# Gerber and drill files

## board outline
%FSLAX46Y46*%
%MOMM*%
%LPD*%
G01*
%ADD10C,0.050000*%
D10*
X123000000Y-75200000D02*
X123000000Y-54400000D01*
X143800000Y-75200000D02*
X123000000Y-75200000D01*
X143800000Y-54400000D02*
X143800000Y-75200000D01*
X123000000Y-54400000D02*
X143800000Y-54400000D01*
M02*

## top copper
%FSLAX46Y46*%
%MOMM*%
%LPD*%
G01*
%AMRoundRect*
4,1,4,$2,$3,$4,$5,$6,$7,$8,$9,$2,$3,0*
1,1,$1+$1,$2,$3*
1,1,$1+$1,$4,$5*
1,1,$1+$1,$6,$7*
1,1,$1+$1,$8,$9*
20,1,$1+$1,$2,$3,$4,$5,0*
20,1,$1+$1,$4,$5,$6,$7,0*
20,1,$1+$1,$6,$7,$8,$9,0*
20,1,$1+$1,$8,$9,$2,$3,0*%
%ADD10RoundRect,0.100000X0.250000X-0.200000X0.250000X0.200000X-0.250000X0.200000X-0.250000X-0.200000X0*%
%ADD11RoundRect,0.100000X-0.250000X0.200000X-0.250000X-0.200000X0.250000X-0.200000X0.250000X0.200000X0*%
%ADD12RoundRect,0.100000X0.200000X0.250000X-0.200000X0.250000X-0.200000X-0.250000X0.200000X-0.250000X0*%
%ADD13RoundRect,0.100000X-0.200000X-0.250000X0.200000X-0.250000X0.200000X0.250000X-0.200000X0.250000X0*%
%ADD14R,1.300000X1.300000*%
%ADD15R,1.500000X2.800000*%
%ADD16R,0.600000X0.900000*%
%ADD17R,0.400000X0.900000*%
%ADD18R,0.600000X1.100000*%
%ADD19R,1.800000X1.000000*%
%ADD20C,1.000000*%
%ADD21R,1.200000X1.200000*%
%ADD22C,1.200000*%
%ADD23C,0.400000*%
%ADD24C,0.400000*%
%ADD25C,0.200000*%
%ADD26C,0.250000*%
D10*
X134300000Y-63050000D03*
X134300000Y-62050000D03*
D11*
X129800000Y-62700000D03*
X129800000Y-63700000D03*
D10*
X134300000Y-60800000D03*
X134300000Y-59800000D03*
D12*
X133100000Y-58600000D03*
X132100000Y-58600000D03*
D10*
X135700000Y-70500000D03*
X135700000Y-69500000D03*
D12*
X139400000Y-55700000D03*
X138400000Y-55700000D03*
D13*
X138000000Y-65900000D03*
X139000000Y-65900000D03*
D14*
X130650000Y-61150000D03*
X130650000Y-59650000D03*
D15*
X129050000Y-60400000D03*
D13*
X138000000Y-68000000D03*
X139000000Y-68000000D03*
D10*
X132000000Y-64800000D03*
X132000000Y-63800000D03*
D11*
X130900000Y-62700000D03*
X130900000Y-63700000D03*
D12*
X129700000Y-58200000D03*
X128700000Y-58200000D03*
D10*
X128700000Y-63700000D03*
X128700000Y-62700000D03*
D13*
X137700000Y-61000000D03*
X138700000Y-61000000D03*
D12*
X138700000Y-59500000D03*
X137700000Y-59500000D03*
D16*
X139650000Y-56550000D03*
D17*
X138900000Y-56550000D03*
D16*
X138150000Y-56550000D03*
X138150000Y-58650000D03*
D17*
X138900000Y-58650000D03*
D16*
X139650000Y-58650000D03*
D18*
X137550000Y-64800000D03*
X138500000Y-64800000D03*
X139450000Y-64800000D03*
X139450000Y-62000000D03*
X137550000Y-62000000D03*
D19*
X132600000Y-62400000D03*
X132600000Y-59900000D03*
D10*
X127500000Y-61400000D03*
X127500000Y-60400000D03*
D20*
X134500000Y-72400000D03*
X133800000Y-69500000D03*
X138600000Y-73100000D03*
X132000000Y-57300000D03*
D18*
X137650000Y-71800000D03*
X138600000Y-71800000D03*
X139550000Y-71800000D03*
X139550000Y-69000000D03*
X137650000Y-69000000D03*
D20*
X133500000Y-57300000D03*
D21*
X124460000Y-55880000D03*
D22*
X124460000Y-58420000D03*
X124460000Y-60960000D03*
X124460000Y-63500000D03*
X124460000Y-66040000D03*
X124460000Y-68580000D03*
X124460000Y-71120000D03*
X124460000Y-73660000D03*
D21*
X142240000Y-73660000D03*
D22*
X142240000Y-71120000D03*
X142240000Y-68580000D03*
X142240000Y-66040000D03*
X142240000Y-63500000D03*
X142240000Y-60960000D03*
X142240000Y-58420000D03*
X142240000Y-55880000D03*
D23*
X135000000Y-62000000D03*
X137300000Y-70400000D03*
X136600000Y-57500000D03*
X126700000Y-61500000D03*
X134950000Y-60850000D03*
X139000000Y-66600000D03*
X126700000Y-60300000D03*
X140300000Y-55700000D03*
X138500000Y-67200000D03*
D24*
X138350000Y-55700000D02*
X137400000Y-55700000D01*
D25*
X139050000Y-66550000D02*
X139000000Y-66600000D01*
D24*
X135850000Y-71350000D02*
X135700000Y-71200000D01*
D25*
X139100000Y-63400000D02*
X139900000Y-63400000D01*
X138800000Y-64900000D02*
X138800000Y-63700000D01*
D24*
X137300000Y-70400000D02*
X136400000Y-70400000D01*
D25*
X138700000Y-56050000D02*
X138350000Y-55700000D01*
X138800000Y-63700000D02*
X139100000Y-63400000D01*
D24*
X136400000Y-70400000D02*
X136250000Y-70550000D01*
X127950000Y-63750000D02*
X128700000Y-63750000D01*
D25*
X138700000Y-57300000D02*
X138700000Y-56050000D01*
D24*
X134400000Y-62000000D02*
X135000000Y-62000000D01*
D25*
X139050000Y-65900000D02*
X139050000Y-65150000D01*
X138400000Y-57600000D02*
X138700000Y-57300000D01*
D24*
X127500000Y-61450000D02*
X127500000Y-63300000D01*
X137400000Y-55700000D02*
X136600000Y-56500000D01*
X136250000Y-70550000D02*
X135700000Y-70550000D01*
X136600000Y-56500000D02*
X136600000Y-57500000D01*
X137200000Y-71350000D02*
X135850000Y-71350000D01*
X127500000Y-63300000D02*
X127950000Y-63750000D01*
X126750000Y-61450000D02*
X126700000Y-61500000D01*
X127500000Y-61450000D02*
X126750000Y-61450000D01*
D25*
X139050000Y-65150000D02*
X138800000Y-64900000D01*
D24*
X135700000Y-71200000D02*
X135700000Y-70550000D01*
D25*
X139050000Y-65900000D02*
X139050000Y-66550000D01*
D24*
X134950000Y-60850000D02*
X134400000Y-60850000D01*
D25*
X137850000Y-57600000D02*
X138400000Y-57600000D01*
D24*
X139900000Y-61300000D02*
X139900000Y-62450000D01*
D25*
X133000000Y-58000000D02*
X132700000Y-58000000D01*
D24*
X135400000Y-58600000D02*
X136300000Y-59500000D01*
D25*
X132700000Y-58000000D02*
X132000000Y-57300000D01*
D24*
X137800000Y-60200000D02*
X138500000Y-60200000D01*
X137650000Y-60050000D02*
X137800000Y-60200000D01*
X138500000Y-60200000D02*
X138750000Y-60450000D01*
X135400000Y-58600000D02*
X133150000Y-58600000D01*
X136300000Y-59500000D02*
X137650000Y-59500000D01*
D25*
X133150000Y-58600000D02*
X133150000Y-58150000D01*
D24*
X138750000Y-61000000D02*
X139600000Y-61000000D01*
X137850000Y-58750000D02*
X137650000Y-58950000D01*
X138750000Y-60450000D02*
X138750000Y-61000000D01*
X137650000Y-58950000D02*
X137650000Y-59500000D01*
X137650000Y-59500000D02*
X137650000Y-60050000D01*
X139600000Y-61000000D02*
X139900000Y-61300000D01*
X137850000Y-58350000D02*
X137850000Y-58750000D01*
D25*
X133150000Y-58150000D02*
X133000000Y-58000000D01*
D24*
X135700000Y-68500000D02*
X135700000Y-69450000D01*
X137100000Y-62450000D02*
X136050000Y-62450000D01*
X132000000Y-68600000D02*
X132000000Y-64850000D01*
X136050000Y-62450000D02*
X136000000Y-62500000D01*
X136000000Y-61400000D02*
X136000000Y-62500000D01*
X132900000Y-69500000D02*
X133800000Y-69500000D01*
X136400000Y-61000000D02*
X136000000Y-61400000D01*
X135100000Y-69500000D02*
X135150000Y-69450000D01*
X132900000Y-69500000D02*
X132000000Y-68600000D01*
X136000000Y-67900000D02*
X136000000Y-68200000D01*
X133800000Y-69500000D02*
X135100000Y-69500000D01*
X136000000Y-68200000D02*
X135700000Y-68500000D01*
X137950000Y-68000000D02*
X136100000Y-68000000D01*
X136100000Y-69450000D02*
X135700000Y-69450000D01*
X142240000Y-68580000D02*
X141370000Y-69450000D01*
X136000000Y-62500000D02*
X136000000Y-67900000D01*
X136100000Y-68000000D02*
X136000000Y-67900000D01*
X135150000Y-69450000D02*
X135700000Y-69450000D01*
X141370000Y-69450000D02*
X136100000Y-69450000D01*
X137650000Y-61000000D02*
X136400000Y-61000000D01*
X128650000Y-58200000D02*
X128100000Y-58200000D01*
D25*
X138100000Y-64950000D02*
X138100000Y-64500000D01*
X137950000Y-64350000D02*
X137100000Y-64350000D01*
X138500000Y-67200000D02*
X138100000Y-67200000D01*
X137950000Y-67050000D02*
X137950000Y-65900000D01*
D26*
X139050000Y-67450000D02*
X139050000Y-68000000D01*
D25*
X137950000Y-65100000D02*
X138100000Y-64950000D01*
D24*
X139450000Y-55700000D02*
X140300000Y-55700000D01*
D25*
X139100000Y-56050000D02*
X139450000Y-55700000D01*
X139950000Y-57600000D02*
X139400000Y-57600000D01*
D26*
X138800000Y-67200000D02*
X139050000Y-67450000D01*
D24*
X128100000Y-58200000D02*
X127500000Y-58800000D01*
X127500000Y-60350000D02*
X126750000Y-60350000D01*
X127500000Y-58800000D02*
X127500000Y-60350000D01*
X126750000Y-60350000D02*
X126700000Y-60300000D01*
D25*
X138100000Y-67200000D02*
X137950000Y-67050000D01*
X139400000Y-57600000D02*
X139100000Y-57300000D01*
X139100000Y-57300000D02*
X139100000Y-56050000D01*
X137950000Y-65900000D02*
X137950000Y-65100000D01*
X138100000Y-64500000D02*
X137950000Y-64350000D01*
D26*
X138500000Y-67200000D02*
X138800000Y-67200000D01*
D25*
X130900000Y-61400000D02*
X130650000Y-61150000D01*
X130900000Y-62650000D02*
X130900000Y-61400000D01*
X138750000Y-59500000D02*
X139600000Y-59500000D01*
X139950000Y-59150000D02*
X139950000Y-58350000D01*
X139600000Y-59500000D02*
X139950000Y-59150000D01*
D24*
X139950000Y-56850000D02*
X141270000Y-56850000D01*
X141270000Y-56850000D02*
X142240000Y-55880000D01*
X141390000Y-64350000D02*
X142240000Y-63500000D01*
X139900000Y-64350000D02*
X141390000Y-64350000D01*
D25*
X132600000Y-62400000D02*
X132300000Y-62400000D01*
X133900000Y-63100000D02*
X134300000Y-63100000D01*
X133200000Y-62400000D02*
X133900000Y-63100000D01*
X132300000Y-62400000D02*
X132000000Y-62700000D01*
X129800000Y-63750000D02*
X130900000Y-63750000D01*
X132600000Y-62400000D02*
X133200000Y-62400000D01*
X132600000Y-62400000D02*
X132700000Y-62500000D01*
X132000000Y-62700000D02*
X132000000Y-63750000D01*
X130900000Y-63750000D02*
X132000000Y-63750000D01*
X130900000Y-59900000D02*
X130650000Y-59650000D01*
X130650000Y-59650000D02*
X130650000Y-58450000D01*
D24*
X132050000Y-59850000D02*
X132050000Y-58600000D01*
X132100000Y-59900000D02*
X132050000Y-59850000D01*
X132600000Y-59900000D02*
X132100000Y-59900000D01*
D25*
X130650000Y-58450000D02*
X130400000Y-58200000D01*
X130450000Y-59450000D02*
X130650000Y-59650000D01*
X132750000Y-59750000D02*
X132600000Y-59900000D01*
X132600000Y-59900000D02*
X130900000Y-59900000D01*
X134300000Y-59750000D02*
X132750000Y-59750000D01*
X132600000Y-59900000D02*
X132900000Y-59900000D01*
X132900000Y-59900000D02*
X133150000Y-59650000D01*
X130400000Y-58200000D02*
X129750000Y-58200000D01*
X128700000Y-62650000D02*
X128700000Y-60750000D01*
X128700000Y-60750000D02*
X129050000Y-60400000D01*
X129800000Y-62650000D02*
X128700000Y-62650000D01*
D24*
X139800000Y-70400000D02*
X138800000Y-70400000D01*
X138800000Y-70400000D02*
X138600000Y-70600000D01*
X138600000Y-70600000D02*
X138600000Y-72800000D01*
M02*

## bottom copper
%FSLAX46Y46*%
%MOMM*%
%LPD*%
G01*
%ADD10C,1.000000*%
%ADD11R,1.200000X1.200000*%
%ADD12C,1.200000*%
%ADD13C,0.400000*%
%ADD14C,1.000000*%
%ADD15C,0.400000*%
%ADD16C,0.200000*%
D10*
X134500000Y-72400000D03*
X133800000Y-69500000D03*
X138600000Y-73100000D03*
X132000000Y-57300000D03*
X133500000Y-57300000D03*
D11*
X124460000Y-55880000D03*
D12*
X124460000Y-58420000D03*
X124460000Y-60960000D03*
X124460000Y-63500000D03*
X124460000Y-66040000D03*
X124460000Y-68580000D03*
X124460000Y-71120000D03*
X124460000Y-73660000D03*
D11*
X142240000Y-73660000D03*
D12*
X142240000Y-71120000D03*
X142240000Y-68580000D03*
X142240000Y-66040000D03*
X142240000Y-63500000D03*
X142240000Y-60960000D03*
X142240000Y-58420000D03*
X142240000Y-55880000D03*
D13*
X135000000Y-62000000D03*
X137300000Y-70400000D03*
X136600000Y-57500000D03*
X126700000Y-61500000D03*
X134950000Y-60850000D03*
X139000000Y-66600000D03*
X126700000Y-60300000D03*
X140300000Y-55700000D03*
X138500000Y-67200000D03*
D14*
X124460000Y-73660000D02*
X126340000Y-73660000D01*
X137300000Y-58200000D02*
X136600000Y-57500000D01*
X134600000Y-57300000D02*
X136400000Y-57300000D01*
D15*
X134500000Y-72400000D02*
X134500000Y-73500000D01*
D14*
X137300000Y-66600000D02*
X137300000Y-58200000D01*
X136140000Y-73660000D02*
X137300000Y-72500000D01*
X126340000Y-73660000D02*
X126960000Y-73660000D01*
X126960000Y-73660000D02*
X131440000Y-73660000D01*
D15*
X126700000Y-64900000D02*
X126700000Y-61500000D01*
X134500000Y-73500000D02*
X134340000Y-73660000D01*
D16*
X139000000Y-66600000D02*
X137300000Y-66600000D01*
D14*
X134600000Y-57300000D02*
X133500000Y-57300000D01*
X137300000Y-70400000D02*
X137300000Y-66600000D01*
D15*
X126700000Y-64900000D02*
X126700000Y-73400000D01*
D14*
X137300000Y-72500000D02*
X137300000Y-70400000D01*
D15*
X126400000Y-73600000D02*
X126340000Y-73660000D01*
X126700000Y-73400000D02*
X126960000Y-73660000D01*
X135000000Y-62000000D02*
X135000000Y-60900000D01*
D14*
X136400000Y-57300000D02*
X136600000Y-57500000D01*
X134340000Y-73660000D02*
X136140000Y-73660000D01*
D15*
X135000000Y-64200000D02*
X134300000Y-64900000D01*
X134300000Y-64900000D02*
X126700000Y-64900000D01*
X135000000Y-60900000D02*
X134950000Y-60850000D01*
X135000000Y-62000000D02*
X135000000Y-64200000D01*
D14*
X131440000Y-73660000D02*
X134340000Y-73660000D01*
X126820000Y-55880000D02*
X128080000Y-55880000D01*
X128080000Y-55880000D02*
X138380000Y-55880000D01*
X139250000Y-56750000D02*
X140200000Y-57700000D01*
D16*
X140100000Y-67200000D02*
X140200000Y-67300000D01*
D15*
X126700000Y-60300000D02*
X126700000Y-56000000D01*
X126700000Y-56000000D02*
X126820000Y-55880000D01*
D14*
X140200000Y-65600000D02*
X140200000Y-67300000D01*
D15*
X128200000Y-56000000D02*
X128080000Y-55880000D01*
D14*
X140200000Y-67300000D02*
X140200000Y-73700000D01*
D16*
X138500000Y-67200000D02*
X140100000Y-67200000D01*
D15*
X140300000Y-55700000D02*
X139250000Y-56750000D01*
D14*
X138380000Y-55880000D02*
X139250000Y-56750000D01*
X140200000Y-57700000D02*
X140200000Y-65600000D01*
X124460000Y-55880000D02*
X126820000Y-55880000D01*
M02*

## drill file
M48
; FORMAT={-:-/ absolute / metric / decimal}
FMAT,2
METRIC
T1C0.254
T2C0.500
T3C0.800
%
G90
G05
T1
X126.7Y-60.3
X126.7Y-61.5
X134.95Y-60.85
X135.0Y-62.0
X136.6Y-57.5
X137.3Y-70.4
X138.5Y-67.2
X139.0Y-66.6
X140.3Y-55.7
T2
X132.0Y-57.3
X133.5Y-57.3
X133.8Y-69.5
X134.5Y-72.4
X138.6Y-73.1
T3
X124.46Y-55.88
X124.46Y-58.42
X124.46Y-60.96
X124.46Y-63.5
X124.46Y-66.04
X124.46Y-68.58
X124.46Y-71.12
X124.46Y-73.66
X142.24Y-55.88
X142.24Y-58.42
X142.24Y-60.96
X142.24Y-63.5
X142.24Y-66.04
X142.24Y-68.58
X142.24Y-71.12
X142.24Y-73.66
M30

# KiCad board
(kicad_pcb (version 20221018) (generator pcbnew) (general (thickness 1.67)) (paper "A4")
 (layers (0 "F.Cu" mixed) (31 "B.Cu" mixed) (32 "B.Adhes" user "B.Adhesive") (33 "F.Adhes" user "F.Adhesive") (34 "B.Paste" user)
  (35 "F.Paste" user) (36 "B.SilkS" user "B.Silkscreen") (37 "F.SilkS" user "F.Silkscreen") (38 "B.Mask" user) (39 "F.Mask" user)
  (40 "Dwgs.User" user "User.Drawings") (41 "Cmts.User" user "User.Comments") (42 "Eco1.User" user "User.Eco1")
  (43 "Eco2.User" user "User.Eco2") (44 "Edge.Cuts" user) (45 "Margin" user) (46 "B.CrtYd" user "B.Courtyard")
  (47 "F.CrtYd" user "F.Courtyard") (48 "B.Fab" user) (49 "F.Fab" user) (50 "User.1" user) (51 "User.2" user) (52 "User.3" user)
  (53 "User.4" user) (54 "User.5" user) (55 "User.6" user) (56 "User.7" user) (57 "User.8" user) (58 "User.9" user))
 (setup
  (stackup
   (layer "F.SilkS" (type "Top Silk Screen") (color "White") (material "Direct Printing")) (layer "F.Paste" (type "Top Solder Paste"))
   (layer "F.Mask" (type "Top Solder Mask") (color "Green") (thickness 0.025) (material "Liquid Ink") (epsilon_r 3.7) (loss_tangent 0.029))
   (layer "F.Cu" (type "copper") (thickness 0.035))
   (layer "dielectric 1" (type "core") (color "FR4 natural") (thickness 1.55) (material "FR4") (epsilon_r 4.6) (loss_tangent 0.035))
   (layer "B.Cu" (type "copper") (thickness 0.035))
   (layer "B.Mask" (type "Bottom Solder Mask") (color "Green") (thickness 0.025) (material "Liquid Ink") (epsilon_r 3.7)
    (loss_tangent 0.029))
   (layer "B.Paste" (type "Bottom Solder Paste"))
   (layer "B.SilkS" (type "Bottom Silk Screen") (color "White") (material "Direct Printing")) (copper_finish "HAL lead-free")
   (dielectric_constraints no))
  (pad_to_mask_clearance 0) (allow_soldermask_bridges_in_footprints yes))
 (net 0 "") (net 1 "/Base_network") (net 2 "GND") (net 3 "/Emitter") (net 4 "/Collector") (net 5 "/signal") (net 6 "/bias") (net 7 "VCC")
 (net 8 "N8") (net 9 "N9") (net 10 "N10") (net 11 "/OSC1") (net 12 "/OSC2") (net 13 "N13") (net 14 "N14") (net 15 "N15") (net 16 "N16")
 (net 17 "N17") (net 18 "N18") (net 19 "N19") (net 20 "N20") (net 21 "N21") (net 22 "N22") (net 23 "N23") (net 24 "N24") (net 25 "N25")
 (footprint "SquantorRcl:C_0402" (layer "F.Cu") (at 134.3 62.55 90)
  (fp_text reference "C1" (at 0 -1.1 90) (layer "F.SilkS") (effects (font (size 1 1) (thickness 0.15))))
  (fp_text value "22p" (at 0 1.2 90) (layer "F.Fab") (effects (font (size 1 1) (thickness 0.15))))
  (pad "1" smd roundrect (at -0.5 0 90) (size 0.6 0.7) (layers "F.Cu" "F.Paste" "F.Mask") (roundrect_rratio 0.1666666667)
   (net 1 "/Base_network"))
  (pad "2" smd roundrect (at 0.5 0 90) (size 0.6 0.7) (layers "F.Cu" "F.Paste" "F.Mask") (roundrect_rratio 0.1666666667) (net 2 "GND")))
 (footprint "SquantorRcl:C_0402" (layer "F.Cu") (at 129.8 63.2 -90)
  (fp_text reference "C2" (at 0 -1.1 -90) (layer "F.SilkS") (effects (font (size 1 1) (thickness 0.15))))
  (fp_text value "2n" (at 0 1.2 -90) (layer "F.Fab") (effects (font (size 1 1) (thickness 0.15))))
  (pad "1" smd roundrect (at -0.5 0 270) (size 0.6 0.7) (layers "F.Cu" "F.Paste" "F.Mask") (roundrect_rratio 0.1666666667)
   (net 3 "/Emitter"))
  (pad "2" smd roundrect (at 0.5 0 270) (size 0.6 0.7) (layers "F.Cu" "F.Paste" "F.Mask") (roundrect_rratio 0.1666666667)
   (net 1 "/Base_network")))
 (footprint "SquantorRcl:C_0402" (layer "F.Cu") (at 134.3 60.3 90)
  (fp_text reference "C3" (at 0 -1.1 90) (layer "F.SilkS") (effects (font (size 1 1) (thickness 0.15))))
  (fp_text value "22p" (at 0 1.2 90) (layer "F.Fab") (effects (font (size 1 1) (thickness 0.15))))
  (pad "1" smd roundrect (at -0.5 0 90) (size 0.6 0.7) (layers "F.Cu" "F.Paste" "F.Mask") (roundrect_rratio 0.1666666667) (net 2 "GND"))
  (pad "2" smd roundrect (at 0.5 0 90) (size 0.6 0.7) (layers "F.Cu" "F.Paste" "F.Mask") (roundrect_rratio 0.1666666667)
   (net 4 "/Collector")))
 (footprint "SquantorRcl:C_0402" (layer "F.Cu") (at 132.6 58.6 180)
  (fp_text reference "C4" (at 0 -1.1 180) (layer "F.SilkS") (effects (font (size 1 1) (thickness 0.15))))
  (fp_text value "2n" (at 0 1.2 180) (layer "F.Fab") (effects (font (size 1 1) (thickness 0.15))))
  (pad "1" smd roundrect (at -0.5 0 180) (size 0.6 0.7) (layers "F.Cu" "F.Paste" "F.Mask") (roundrect_rratio 0.1666666667) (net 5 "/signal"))
  (pad "2" smd roundrect (at 0.5 0 180) (size 0.6 0.7) (layers "F.Cu" "F.Paste" "F.Mask") (roundrect_rratio 0.1666666667)
   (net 4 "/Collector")))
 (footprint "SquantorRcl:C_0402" (layer "F.Cu") (at 135.7 70 90)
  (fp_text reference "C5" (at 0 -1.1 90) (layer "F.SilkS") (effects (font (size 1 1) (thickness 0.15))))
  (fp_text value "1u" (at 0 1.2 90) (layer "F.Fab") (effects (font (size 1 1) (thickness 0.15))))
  (pad "1" smd roundrect (at -0.5 0 90) (size 0.6 0.7) (layers "F.Cu" "F.Paste" "F.Mask") (roundrect_rratio 0.1666666667) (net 2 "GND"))
  (pad "2" smd roundrect (at 0.5 0 90) (size 0.6 0.7) (layers "F.Cu" "F.Paste" "F.Mask") (roundrect_rratio 0.1666666667) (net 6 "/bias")))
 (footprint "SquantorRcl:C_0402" (layer "F.Cu") (at 138.9 55.7 180)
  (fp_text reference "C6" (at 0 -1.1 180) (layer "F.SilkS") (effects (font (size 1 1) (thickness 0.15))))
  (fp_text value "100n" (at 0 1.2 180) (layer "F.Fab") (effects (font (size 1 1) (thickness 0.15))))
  (pad "1" smd roundrect (at -0.5 0 180) (size 0.6 0.7) (layers "F.Cu" "F.Paste" "F.Mask") (roundrect_rratio 0.1666666667) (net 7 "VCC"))
  (pad "2" smd roundrect (at 0.5 0 180) (size 0.6 0.7) (layers "F.Cu" "F.Paste" "F.Mask") (roundrect_rratio 0.1666666667) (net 2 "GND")))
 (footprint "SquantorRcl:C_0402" (layer "F.Cu") (at 138.5 65.9)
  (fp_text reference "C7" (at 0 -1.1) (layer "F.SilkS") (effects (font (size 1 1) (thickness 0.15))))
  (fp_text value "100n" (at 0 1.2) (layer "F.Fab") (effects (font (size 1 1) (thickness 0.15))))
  (pad "1" smd roundrect (at -0.5 0) (size 0.6 0.7) (layers "F.Cu" "F.Paste" "F.Mask") (roundrect_rratio 0.1666666667) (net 7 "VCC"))
  (pad "2" smd roundrect (at 0.5 0) (size 0.6 0.7) (layers "F.Cu" "F.Paste" "F.Mask") (roundrect_rratio 0.1666666667) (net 2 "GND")))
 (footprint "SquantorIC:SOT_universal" (layer "F.Cu") (at 129.9 60.4 90)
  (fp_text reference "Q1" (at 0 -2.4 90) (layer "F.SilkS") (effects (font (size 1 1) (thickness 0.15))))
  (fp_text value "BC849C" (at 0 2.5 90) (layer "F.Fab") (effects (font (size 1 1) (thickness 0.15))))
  (pad "1" smd rect (at -0.75 0.75 90) (size 1.3 1.3) (layers "F.Cu" "F.Paste" "F.Mask") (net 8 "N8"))
  (pad "2" smd rect (at 0.75 0.75 90) (size 1.3 1.3) (layers "F.Cu" "F.Paste" "F.Mask") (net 4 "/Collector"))
  (pad "3" smd rect (at 0 -0.85 90) (size 2.8 1.5) (layers "F.Cu" "F.Paste" "F.Mask") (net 3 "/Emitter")))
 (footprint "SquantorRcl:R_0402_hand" (layer "F.Cu") (at 138.5 68)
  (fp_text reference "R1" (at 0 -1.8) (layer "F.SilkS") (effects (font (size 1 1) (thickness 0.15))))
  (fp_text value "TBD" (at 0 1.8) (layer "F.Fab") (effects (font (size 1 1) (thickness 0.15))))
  (pad "1" smd roundrect (at -0.5 0) (size 0.6 0.7) (layers "F.Cu" "F.Paste" "F.Mask") (roundrect_rratio 0.1666666667) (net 6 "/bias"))
  (pad "2" smd roundrect (at 0.5 0) (size 0.6 0.7) (layers "F.Cu" "F.Paste" "F.Mask") (roundrect_rratio 0.1666666667) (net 7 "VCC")))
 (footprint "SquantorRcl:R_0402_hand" (layer "F.Cu") (at 132 64.3 90)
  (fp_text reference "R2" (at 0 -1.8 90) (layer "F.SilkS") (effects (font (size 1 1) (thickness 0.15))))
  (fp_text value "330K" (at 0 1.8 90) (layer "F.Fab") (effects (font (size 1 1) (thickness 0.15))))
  (pad "1" smd roundrect (at -0.5 0 90) (size 0.6 0.7) (layers "F.Cu" "F.Paste" "F.Mask") (roundrect_rratio 0.1666666667) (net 6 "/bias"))
  (pad "2" smd roundrect (at 0.5 0 90) (size 0.6 0.7) (layers "F.Cu" "F.Paste" "F.Mask") (roundrect_rratio 0.1666666667)
   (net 1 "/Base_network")))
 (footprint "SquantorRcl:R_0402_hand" (layer "F.Cu") (at 130.9 63.2 -90)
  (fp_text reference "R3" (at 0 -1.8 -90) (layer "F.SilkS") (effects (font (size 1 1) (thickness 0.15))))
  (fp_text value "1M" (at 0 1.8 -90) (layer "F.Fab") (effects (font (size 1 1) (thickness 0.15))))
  (pad "1" smd roundrect (at -0.5 0 270) (size 0.6 0.7) (layers "F.Cu" "F.Paste" "F.Mask") (roundrect_rratio 0.1666666667) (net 8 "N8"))
  (pad "2" smd roundrect (at 0.5 0 270) (size 0.6 0.7) (layers "F.Cu" "F.Paste" "F.Mask") (roundrect_rratio 0.1666666667)
   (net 1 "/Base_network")))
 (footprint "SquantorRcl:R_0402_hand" (layer "F.Cu") (at 129.2 58.2 180)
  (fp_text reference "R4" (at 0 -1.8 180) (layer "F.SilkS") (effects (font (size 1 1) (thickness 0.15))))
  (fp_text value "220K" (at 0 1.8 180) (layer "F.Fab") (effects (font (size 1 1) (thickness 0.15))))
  (pad "1" smd roundrect (at -0.5 0 180) (size 0.6 0.7) (layers "F.Cu" "F.Paste" "F.Mask") (roundrect_rratio 0.1666666667)
   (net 4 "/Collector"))
  (pad "2" smd roundrect (at 0.5 0 180) (size 0.6 0.7) (layers "F.Cu" "F.Paste" "F.Mask") (roundrect_rratio 0.1666666667) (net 7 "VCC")))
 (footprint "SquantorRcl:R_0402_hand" (layer "F.Cu") (at 128.7 63.2 90)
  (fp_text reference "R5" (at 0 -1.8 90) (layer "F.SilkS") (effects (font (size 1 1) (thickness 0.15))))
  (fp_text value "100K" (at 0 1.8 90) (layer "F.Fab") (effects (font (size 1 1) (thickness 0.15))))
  (pad "1" smd roundrect (at -0.5 0 90) (size 0.6 0.7) (layers "F.Cu" "F.Paste" "F.Mask") (roundrect_rratio 0.1666666667) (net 2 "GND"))
  (pad "2" smd roundrect (at 0.5 0 90) (size 0.6 0.7) (layers "F.Cu" "F.Paste" "F.Mask") (roundrect_rratio 0.1666666667) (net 3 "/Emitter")))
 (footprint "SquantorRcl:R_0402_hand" (layer "F.Cu") (at 138.2 61)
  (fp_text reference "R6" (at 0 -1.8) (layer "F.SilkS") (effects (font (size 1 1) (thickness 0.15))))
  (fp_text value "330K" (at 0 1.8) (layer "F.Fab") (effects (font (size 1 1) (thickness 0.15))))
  (pad "1" smd roundrect (at -0.5 0) (size 0.6 0.7) (layers "F.Cu" "F.Paste" "F.Mask") (roundrect_rratio 0.1666666667) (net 6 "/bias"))
  (pad "2" smd roundrect (at 0.5 0) (size 0.6 0.7) (layers "F.Cu" "F.Paste" "F.Mask") (roundrect_rratio 0.1666666667) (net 5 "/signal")))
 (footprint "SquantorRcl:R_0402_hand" (layer "F.Cu") (at 138.2 59.5 180)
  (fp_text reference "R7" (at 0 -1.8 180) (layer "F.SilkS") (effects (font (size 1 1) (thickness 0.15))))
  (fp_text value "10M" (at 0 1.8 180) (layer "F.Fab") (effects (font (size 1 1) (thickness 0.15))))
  (pad "1" smd roundrect (at -0.5 0 180) (size 0.6 0.7) (layers "F.Cu" "F.Paste" "F.Mask") (roundrect_rratio 0.1666666667) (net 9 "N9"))
  (pad "2" smd roundrect (at 0.5 0 180) (size 0.6 0.7) (layers "F.Cu" "F.Paste" "F.Mask") (roundrect_rratio 0.1666666667) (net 5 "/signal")))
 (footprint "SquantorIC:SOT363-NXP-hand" (layer "F.Cu") (at 138.9 57.6 -90)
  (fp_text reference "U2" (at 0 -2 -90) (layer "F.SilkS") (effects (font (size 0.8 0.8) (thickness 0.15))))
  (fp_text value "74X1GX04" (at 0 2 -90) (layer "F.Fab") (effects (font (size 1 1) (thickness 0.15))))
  (pad "1" smd rect (at -1.05 -0.75 180) (size 0.6 0.9) (layers "F.Cu" "F.Paste" "F.Mask") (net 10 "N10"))
  (pad "2" smd rect (at -1.05 0 180) (size 0.4 0.9) (layers "F.Cu" "F.Paste" "F.Mask") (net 2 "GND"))
  (pad "3" smd rect (at -1.05 0.75 180) (size 0.6 0.9) (layers "F.Cu" "F.Paste" "F.Mask") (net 5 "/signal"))
  (pad "4" smd rect (at 1.05 0.75 180) (size 0.6 0.9) (layers "F.Cu" "F.Paste" "F.Mask") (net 9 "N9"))
  (pad "5" smd rect (at 1.05 0 180) (size 0.4 0.9) (layers "F.Cu" "F.Paste" "F.Mask") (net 7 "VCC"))
  (pad "6" smd rect (at 1.05 -0.75 180) (size 0.6 0.9) (layers "F.Cu" "F.Paste" "F.Mask") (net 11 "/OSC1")))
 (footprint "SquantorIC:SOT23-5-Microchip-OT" (layer "F.Cu") (at 138.5 63.4 90)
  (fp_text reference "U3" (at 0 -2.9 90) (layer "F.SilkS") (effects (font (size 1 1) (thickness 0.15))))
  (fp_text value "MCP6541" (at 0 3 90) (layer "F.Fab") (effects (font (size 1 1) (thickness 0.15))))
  (pad "1" smd rect (at -1.4 -0.95) (size 0.6 1.1) (layers "F.Cu" "F.Paste" "F.Mask") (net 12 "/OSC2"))
  (pad "2" smd rect (at -1.4 0) (size 0.6 1.1) (layers "F.Cu" "F.Paste" "F.Mask") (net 2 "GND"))
  (pad "3" smd rect (at -1.4 0.95) (size 0.6 1.1) (layers "F.Cu" "F.Paste" "F.Mask") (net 5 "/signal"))
  (pad "4" smd rect (at 1.4 0.95) (size 0.6 1.1) (layers "F.Cu" "F.Paste" "F.Mask") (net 6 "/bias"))
  (pad "5" smd rect (at 1.4 -0.95) (size 0.6 1.1) (layers "F.Cu" "F.Paste" "F.Mask") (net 7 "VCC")))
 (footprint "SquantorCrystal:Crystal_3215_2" (layer "F.Cu") (at 132.6 61.15 90)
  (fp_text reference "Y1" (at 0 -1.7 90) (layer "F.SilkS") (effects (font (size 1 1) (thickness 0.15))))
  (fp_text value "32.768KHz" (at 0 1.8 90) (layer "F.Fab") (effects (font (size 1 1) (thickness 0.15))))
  (pad "1" smd rect (at -1.25 0 90) (size 1 1.8) (layers "F.Cu" "F.Paste" "F.Mask") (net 1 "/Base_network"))
  (pad "2" smd rect (at 1.25 0 90) (size 1 1.8) (layers "F.Cu" "F.Paste" "F.Mask") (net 4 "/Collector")))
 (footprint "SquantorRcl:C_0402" (layer "F.Cu") (at 127.5 60.9 90)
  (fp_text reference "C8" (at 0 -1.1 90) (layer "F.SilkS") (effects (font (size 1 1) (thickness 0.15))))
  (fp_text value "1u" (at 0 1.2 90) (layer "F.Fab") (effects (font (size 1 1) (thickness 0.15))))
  (pad "1" smd roundrect (at -0.5 0 90) (size 0.6 0.7) (layers "F.Cu" "F.Paste" "F.Mask") (roundrect_rratio 0.1666666667) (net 2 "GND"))
  (pad "2" smd roundrect (at 0.5 0 90) (size 0.6 0.7) (layers "F.Cu" "F.Paste" "F.Mask") (roundrect_rratio 0.1666666667) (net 7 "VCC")))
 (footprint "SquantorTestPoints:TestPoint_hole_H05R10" (layer "F.Cu") (at 134.5 72.4)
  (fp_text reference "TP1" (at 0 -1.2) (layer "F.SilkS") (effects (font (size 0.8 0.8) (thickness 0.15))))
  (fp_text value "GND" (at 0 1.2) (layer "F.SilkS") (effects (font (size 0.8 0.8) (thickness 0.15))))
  (pad "1" thru_hole circle (at 0 0) (size 1 1) (drill 0.5) (layers "*.Cu" "*.Mask") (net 2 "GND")))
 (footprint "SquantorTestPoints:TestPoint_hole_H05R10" (layer "F.Cu") (at 133.8 69.5)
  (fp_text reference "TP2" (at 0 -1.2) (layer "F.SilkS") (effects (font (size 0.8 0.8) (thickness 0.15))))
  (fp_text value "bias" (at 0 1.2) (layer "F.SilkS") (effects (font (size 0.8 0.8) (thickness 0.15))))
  (pad "1" thru_hole circle (at 0 0) (size 1 1) (drill 0.5) (layers "*.Cu" "*.Mask") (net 6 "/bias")))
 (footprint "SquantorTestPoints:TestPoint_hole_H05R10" (layer "F.Cu") (at 138.6 73.1)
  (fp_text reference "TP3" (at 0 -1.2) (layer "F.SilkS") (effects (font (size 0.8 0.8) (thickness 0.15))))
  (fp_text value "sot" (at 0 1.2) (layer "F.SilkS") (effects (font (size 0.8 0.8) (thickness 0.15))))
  (pad "1" thru_hole circle (at 0 0) (size 1 1) (drill 0.5) (layers "*.Cu" "*.Mask") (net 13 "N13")))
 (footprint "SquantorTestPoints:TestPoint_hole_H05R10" (layer "F.Cu") (at 132 57.3)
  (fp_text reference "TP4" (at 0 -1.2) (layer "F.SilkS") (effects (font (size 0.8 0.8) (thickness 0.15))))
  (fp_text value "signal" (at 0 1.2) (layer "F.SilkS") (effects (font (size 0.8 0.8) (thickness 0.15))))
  (pad "1" thru_hole circle (at 0 0) (size 1 1) (drill 0.5) (layers "*.Cu" "*.Mask") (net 5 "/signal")))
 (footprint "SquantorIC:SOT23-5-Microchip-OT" (layer "F.Cu") (at 138.6 70.4 90)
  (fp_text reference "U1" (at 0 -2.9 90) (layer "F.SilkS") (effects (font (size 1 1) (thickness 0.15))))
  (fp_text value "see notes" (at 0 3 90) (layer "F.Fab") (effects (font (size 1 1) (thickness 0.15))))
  (pad "1" smd rect (at -1.4 -0.95) (size 0.6 1.1) (layers "F.Cu" "F.Paste" "F.Mask") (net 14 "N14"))
  (pad "2" smd rect (at -1.4 0) (size 0.6 1.1) (layers "F.Cu" "F.Paste" "F.Mask") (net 13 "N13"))
  (pad "3" smd rect (at -1.4 0.95) (size 0.6 1.1) (layers "F.Cu" "F.Paste" "F.Mask") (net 6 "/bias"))
  (pad "4" smd rect (at 1.4 0.95) (size 0.6 1.1) (layers "F.Cu" "F.Paste" "F.Mask") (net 6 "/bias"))
  (pad "5" smd rect (at 1.4 -0.95) (size 0.6 1.1) (layers "F.Cu" "F.Paste" "F.Mask") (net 2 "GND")))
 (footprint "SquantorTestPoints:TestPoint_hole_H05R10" (layer "F.Cu") (at 133.5 57.3)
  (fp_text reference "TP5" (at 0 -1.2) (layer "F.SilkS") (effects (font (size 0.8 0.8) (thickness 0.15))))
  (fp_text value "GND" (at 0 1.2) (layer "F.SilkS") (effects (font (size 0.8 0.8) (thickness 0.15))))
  (pad "1" thru_hole circle (at 0 0) (size 1 1) (drill 0.5) (layers "*.Cu" "*.Mask") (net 2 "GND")))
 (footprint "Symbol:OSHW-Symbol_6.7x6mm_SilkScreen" (layer "B.Cu") (at 134.27 64.77 180)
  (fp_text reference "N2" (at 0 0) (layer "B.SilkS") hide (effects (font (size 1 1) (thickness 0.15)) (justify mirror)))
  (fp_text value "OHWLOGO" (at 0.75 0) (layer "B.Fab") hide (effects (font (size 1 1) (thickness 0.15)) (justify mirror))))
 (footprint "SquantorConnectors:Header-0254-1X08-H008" (layer "B.Cu") (at 124.46 64.77 -90)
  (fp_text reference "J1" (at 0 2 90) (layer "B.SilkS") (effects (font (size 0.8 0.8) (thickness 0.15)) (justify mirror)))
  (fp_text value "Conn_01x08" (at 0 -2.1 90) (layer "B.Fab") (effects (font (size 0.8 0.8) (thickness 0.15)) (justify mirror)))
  (pad "1" thru_hole rect (at -8.89 0 90) (size 1.2 1.2) (drill 0.8) (layers "*.Cu" "*.Mask") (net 7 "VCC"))
  (pad "2" thru_hole circle (at -6.35 0 90) (size 1.2 1.2) (drill 0.8) (layers "*.Cu" "*.Mask") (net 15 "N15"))
  (pad "3" thru_hole circle (at -3.81 0 90) (size 1.2 1.2) (drill 0.8) (layers "*.Cu" "*.Mask") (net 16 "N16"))
  (pad "4" thru_hole circle (at -1.27 0 90) (size 1.2 1.2) (drill 0.8) (layers "*.Cu" "*.Mask") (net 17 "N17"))
  (pad "5" thru_hole circle (at 1.27 0 90) (size 1.2 1.2) (drill 0.8) (layers "*.Cu" "*.Mask") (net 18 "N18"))
  (pad "6" thru_hole circle (at 3.81 0 90) (size 1.2 1.2) (drill 0.8) (layers "*.Cu" "*.Mask") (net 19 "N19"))
  (pad "7" thru_hole circle (at 6.35 0 90) (size 1.2 1.2) (drill 0.8) (layers "*.Cu" "*.Mask") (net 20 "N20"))
  (pad "8" thru_hole circle (at 8.89 0 90) (size 1.2 1.2) (drill 0.8) (layers "*.Cu" "*.Mask") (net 2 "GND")))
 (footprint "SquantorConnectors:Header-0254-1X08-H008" (layer "B.Cu") (at 142.24 64.77 90)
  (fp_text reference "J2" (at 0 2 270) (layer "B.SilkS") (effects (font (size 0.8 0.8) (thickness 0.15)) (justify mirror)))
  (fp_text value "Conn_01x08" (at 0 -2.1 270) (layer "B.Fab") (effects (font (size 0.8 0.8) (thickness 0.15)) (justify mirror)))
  (pad "1" thru_hole rect (at -8.89 0 270) (size 1.2 1.2) (drill 0.8) (layers "*.Cu" "*.Mask") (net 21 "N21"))
  (pad "2" thru_hole circle (at -6.35 0 270) (size 1.2 1.2) (drill 0.8) (layers "*.Cu" "*.Mask") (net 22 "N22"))
  (pad "3" thru_hole circle (at -3.81 0 270) (size 1.2 1.2) (drill 0.8) (layers "*.Cu" "*.Mask") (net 6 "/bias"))
  (pad "4" thru_hole circle (at -1.27 0 270) (size 1.2 1.2) (drill 0.8) (layers "*.Cu" "*.Mask") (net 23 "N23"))
  (pad "5" thru_hole circle (at 1.27 0 270) (size 1.2 1.2) (drill 0.8) (layers "*.Cu" "*.Mask") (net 12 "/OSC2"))
  (pad "6" thru_hole circle (at 3.81 0 270) (size 1.2 1.2) (drill 0.8) (layers "*.Cu" "*.Mask") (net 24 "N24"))
  (pad "7" thru_hole circle (at 6.35 0 270) (size 1.2 1.2) (drill 0.8) (layers "*.Cu" "*.Mask") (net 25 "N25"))
  (pad "8" thru_hole circle (at 8.89 0 270) (size 1.2 1.2) (drill 0.8) (layers "*.Cu" "*.Mask") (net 11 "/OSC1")))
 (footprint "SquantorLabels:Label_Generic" (layer "B.Cu") (at 134.97 68.3 180)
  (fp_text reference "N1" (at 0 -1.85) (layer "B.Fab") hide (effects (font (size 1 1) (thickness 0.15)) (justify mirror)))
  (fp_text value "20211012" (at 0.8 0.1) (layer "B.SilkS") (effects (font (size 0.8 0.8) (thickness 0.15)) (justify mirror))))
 (gr_line (start 123 75.2) (end 123 54.4) (stroke (width 0.05) (type solid)) (layer "Edge.Cuts"))
 (gr_line (start 143.8 75.2) (end 123 75.2) (stroke (width 0.05) (type solid)) (layer "Edge.Cuts"))
 (gr_line (start 143.8 54.4) (end 143.8 75.2) (stroke (width 0.05) (type solid)) (layer "Edge.Cuts"))
 (gr_line (start 123 54.4) (end 143.8 54.4) (stroke (width 0.05) (type solid)) (layer "Edge.Cuts"))
 (segment (start 138.35 55.7) (end 137.4 55.7) (width 0.4) (layer "F.Cu") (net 2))
 (segment (start 139.05 66.55) (end 139 66.6) (width 0.2) (layer "F.Cu") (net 2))
 (segment (start 135.85 71.35) (end 135.7 71.2) (width 0.4) (layer "F.Cu") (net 2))
 (segment (start 139.1 63.4) (end 139.9 63.4) (width 0.2) (layer "F.Cu") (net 2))
 (segment (start 138.8 64.9) (end 138.8 63.7) (width 0.2) (layer "F.Cu") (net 2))
 (segment (start 137.3 70.4) (end 136.4 70.4) (width 0.4) (layer "F.Cu") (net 2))
 (segment (start 138.7 56.05) (end 138.35 55.7) (width 0.2) (layer "F.Cu") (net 2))
 (segment (start 138.8 63.7) (end 139.1 63.4) (width 0.2) (layer "F.Cu") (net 2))
 (segment (start 136.4 70.4) (end 136.25 70.55) (width 0.4) (layer "F.Cu") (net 2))
 (segment (start 127.95 63.75) (end 128.7 63.75) (width 0.4) (layer "F.Cu") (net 2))
 (segment (start 138.7 57.3) (end 138.7 56.05) (width 0.2) (layer "F.Cu") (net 2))
 (segment (start 134.4 62) (end 135 62) (width 0.4) (layer "F.Cu") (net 2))
 (segment (start 139.05 65.9) (end 139.05 65.15) (width 0.2) (layer "F.Cu") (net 2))
 (segment (start 138.4 57.6) (end 138.7 57.3) (width 0.2) (layer "F.Cu") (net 2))
 (segment (start 127.5 61.45) (end 127.5 63.3) (width 0.4) (layer "F.Cu") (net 2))
 (segment (start 137.4 55.7) (end 136.6 56.5) (width 0.4) (layer "F.Cu") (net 2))
 (segment (start 136.25 70.55) (end 135.7 70.55) (width 0.4) (layer "F.Cu") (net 2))
 (segment (start 136.6 56.5) (end 136.6 57.5) (width 0.4) (layer "F.Cu") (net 2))
 (segment (start 137.2 71.35) (end 135.85 71.35) (width 0.4) (layer "F.Cu") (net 2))
 (segment (start 127.5 63.3) (end 127.95 63.75) (width 0.4) (layer "F.Cu") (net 2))
 (segment (start 126.75 61.45) (end 126.7 61.5) (width 0.4) (layer "F.Cu") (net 2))
 (segment (start 127.5 61.45) (end 126.75 61.45) (width 0.4) (layer "F.Cu") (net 2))
 (segment (start 139.05 65.15) (end 138.8 64.9) (width 0.2) (layer "F.Cu") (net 2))
 (segment (start 135.7 71.2) (end 135.7 70.55) (width 0.4) (layer "F.Cu") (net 2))
 (segment (start 139.05 65.9) (end 139.05 66.55) (width 0.2) (layer "F.Cu") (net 2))
 (segment (start 134.95 60.85) (end 134.4 60.85) (width 0.4) (layer "F.Cu") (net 2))
 (segment (start 137.85 57.6) (end 138.4 57.6) (width 0.2) (layer "F.Cu") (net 2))
 (via (at 135 62) (size 0.4) (drill 0.254) (layers "F.Cu" "B.Cu") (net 2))
 (via (at 137.3 70.4) (size 0.4) (drill 0.254) (layers "F.Cu" "B.Cu") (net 2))
 (via (at 136.6 57.5) (size 0.4) (drill 0.254) (layers "F.Cu" "B.Cu") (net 2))
 (via (at 126.7 61.5) (size 0.4) (drill 0.254) (layers "F.Cu" "B.Cu") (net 2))
 (via (at 134.95 60.85) (size 0.4) (drill 0.254) (layers "F.Cu" "B.Cu") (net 2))
 (via (at 139 66.6) (size 0.4) (drill 0.254) (layers "F.Cu" "B.Cu") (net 2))
 (segment (start 124.46 73.66) (end 126.34 73.66) (width 1) (layer "B.Cu") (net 2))
 (segment (start 137.3 58.2) (end 136.6 57.5) (width 1) (layer "B.Cu") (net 2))
 (segment (start 134.6 57.3) (end 136.4 57.3) (width 1) (layer "B.Cu") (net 2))
 (segment (start 134.5 72.4) (end 134.5 73.5) (width 0.4) (layer "B.Cu") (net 2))
 (segment (start 137.3 66.6) (end 137.3 58.2) (width 1) (layer "B.Cu") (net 2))
 (segment (start 136.14 73.66) (end 137.3 72.5) (width 1) (layer "B.Cu") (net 2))
 (segment (start 126.34 73.66) (end 126.96 73.66) (width 1) (layer "B.Cu") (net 2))
 (segment (start 126.96 73.66) (end 131.44 73.66) (width 1) (layer "B.Cu") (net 2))
 (segment (start 126.7 64.9) (end 126.7 61.5) (width 0.4) (layer "B.Cu") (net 2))
 (segment (start 134.5 73.5) (end 134.34 73.66) (width 0.4) (layer "B.Cu") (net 2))
 (segment (start 139 66.6) (end 137.3 66.6) (width 0.2) (layer "B.Cu") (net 2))
 (segment (start 134.6 57.3) (end 133.5 57.3) (width 1) (layer "B.Cu") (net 2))
 (segment (start 137.3 70.4) (end 137.3 66.6) (width 1) (layer "B.Cu") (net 2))
 (segment (start 126.7 64.9) (end 126.7 73.4) (width 0.4) (layer "B.Cu") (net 2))
 (segment (start 137.3 72.5) (end 137.3 70.4) (width 1) (layer "B.Cu") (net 2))
 (segment (start 126.4 73.6) (end 126.34 73.66) (width 0.4) (layer "B.Cu") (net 2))
 (segment (start 126.7 73.4) (end 126.96 73.66) (width 0.4) (layer "B.Cu") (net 2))
 (segment (start 135 62) (end 135 60.9) (width 0.4) (layer "B.Cu") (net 2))
 (segment (start 136.4 57.3) (end 136.6 57.5) (width 1) (layer "B.Cu") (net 2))
 (segment (start 134.34 73.66) (end 136.14 73.66) (width 1) (layer "B.Cu") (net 2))
 (segment (start 135 64.2) (end 134.3 64.9) (width 0.4) (layer "B.Cu") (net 2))
 (segment (start 134.3 64.9) (end 126.7 64.9) (width 0.4) (layer "B.Cu") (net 2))
 (segment (start 135 60.9) (end 134.95 60.85) (width 0.4) (layer "B.Cu") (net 2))
 (segment (start 135 62) (end 135 64.2) (width 0.4) (layer "B.Cu") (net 2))
 (segment (start 131.44 73.66) (end 134.34 73.66) (width 1) (layer "B.Cu") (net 2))
 (segment (start 139.9 61.3) (end 139.9 62.45) (width 0.4) (layer "F.Cu") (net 5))
 (segment (start 133 58) (end 132.7 58) (width 0.2) (layer "F.Cu") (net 5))
 (segment (start 135.4 58.6) (end 136.3 59.5) (width 0.4) (layer "F.Cu") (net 5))
 (segment (start 132.7 58) (end 132 57.3) (width 0.2) (layer "F.Cu") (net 5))
 (segment (start 137.8 60.2) (end 138.5 60.2) (width 0.4) (layer "F.Cu") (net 5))
 (segment (start 137.65 60.05) (end 137.8 60.2) (width 0.4) (layer "F.Cu") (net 5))
 (segment (start 138.5 60.2) (end 138.75 60.45) (width 0.4) (layer "F.Cu") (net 5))
 (segment (start 135.4 58.6) (end 133.15 58.6) (width 0.4) (layer "F.Cu") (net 5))
 (segment (start 136.3 59.5) (end 137.65 59.5) (width 0.4) (layer "F.Cu") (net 5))
 (segment (start 133.15 58.6) (end 133.15 58.15) (width 0.2) (layer "F.Cu") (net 5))
 (segment (start 138.75 61) (end 139.6 61) (width 0.4) (layer "F.Cu") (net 5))
 (segment (start 137.85 58.75) (end 137.65 58.95) (width 0.4) (layer "F.Cu") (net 5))
 (segment (start 138.75 60.45) (end 138.75 61) (width 0.4) (layer "F.Cu") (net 5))
 (segment (start 137.65 58.95) (end 137.65 59.5) (width 0.4) (layer "F.Cu") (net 5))
 (segment (start 137.65 59.5) (end 137.65 60.05) (width 0.4) (layer "F.Cu") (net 5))
 (segment (start 139.6 61) (end 139.9 61.3) (width 0.4) (layer "F.Cu") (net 5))
 (segment (start 137.85 58.35) (end 137.85 58.75) (width 0.4) (layer "F.Cu") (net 5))
 (segment (start 133.15 58.15) (end 133 58) (width 0.2) (layer "F.Cu") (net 5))
 (segment (start 135.7 68.5) (end 135.7 69.45) (width 0.4) (layer "F.Cu") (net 6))
 (segment (start 137.1 62.45) (end 136.05 62.45) (width 0.4) (layer "F.Cu") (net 6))
 (segment (start 132 68.6) (end 132 64.85) (width 0.4) (layer "F.Cu") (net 6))
 (segment (start 136.05 62.45) (end 136 62.5) (width 0.4) (layer "F.Cu") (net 6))
 (segment (start 136 61.4) (end 136 62.5) (width 0.4) (layer "F.Cu") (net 6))
 (segment (start 132.9 69.5) (end 133.8 69.5) (width 0.4) (layer "F.Cu") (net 6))
 (segment (start 136.4 61) (end 136 61.4) (width 0.4) (layer "F.Cu") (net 6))
 (segment (start 135.1 69.5) (end 135.15 69.45) (width 0.4) (layer "F.Cu") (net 6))
 (segment (start 132.9 69.5) (end 132 68.6) (width 0.4) (layer "F.Cu") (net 6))
 (segment (start 136 67.9) (end 136 68.2) (width 0.4) (layer "F.Cu") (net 6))
 (segment (start 133.8 69.5) (end 135.1 69.5) (width 0.4) (layer "F.Cu") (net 6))
 (segment (start 136 68.2) (end 135.7 68.5) (width 0.4) (layer "F.Cu") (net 6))
 (segment (start 137.95 68) (end 136.1 68) (width 0.4) (layer "F.Cu") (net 6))
 (segment (start 136.1 69.45) (end 135.7 69.45) (width 0.4) (layer "F.Cu") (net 6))
 (segment (start 142.24 68.58) (end 141.37 69.45) (width 0.4) (layer "F.Cu") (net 6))
 (segment (start 136 62.5) (end 136 67.9) (width 0.4) (layer "F.Cu") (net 6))
 (segment (start 136.1 68) (end 136 67.9) (width 0.4) (layer "F.Cu") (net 6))
 (segment (start 135.15 69.45) (end 135.7 69.45) (width 0.4) (layer "F.Cu") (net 6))
 (segment (start 141.37 69.45) (end 136.1 69.45) (width 0.4) (layer "F.Cu") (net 6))
 (segment (start 137.65 61) (end 136.4 61) (width 0.4) (layer "F.Cu") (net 6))
 (segment (start 128.65 58.2) (end 128.1 58.2) (width 0.4) (layer "F.Cu") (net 7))
 (segment (start 138.1 64.95) (end 138.1 64.5) (width 0.2) (layer "F.Cu") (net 7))
 (segment (start 137.95 64.35) (end 137.1 64.35) (width 0.2) (layer "F.Cu") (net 7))
 (segment (start 138.5 67.2) (end 138.1 67.2) (width 0.2) (layer "F.Cu") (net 7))
 (segment (start 137.95 67.05) (end 137.95 65.9) (width 0.2) (layer "F.Cu") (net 7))
 (segment (start 139.05 67.45) (end 139.05 68) (width 0.25) (layer "F.Cu") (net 7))
 (segment (start 137.95 65.1) (end 138.1 64.95) (width 0.2) (layer "F.Cu") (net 7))
 (segment (start 139.45 55.7) (end 140.3 55.7) (width 0.4) (layer "F.Cu") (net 7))
 (segment (start 139.1 56.05) (end 139.45 55.7) (width 0.2) (layer "F.Cu") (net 7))
 (segment (start 139.95 57.6) (end 139.4 57.6) (width 0.2) (layer "F.Cu") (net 7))
 (segment (start 138.8 67.2) (end 139.05 67.45) (width 0.25) (layer "F.Cu") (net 7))
 (segment (start 128.1 58.2) (end 127.5 58.8) (width 0.4) (layer "F.Cu") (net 7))
 (segment (start 127.5 60.35) (end 126.75 60.35) (width 0.4) (layer "F.Cu") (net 7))
 (segment (start 127.5 58.8) (end 127.5 60.35) (width 0.4) (layer "F.Cu") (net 7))
 (segment (start 126.75 60.35) (end 126.7 60.3) (width 0.4) (layer "F.Cu") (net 7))
 (segment (start 138.1 67.2) (end 137.95 67.05) (width 0.2) (layer "F.Cu") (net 7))
 (segment (start 139.4 57.6) (end 139.1 57.3) (width 0.2) (layer "F.Cu") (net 7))
 (segment (start 139.1 57.3) (end 139.1 56.05) (width 0.2) (layer "F.Cu") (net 7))
 (segment (start 137.95 65.9) (end 137.95 65.1) (width 0.2) (layer "F.Cu") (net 7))
 (segment (start 138.1 64.5) (end 137.95 64.35) (width 0.2) (layer "F.Cu") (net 7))
 (segment (start 138.5 67.2) (end 138.8 67.2) (width 0.25) (layer "F.Cu") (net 7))
 (via (at 126.7 60.3) (size 0.4) (drill 0.254) (layers "F.Cu" "B.Cu") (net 7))
 (via (at 140.3 55.7) (size 0.4) (drill 0.254) (layers "F.Cu" "B.Cu") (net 7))
 (via (at 138.5 67.2) (size 0.4) (drill 0.254) (layers "F.Cu" "B.Cu") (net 7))
 (segment (start 126.82 55.88) (end 128.08 55.88) (width 1) (layer "B.Cu") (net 7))
 (segment (start 128.08 55.88) (end 138.38 55.88) (width 1) (layer "B.Cu") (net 7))
 (segment (start 139.25 56.75) (end 140.2 57.7) (width 1) (layer "B.Cu") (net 7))
 (segment (start 140.1 67.2) (end 140.2 67.3) (width 0.2) (layer "B.Cu") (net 7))
 (segment (start 126.7 60.3) (end 126.7 56) (width 0.4) (layer "B.Cu") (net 7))
 (segment (start 126.7 56) (end 126.82 55.88) (width 0.4) (layer "B.Cu") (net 7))
 (segment (start 140.2 65.6) (end 140.2 67.3) (width 1) (layer "B.Cu") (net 7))
 (segment (start 128.2 56) (end 128.08 55.88) (width 0.4) (layer "B.Cu") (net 7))
 (segment (start 140.2 67.3) (end 140.2 73.7) (width 1) (layer "B.Cu") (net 7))
 (segment (start 138.5 67.2) (end 140.1 67.2) (width 0.2) (layer "B.Cu") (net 7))
 (segment (start 140.3 55.7) (end 139.25 56.75) (width 0.4) (layer "B.Cu") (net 7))
 (segment (start 138.38 55.88) (end 139.25 56.75) (width 1) (layer "B.Cu") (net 7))
 (segment (start 140.2 57.7) (end 140.2 65.6) (width 1) (layer "B.Cu") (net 7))
 (segment (start 124.46 55.88) (end 126.82 55.88) (width 1) (layer "B.Cu") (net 7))
 (segment (start 130.9 61.4) (end 130.65 61.15) (width 0.2) (layer "F.Cu") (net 8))
 (segment (start 130.9 62.65) (end 130.9 61.4) (width 0.2) (layer "F.Cu") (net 8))
 (segment (start 138.75 59.5) (end 139.6 59.5) (width 0.2) (layer "F.Cu") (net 9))
 (segment (start 139.95 59.15) (end 139.95 58.35) (width 0.2) (layer "F.Cu") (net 9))
 (segment (start 139.6 59.5) (end 139.95 59.15) (width 0.2) (layer "F.Cu") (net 9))
 (segment (start 139.95 56.85) (end 141.27 56.85) (width 0.4) (layer "F.Cu") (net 11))
 (segment (start 141.27 56.85) (end 142.24 55.88) (width 0.4) (layer "F.Cu") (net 11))
 (segment (start 141.39 64.35) (end 142.24 63.5) (width 0.4) (layer "F.Cu") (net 12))
 (segment (start 139.9 64.35) (end 141.39 64.35) (width 0.4) (layer "F.Cu") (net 12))
 (segment (start 132.6 62.4) (end 132.3 62.4) (width 0.2) (layer "F.Cu") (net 1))
 (segment (start 133.9 63.1) (end 134.3 63.1) (width 0.2) (layer "F.Cu") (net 1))
 (segment (start 133.2 62.4) (end 133.9 63.1) (width 0.2) (layer "F.Cu") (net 1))
 (segment (start 132.3 62.4) (end 132 62.7) (width 0.2) (layer "F.Cu") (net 1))
 (segment (start 129.8 63.75) (end 130.9 63.75) (width 0.2) (layer "F.Cu") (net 1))
 (segment (start 132.6 62.4) (end 133.2 62.4) (width 0.2) (layer "F.Cu") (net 1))
 (segment (start 132.6 62.4) (end 132.7 62.5) (width 0.2) (layer "F.Cu") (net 1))
 (segment (start 132 62.7) (end 132 63.75) (width 0.2) (layer "F.Cu") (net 1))
 (segment (start 130.9 63.75) (end 132 63.75) (width 0.2) (layer "F.Cu") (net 1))
 (segment (start 130.9 59.9) (end 130.65 59.65) (width 0.2) (layer "F.Cu") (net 4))
 (segment (start 130.65 59.65) (end 130.65 58.45) (width 0.2) (layer "F.Cu") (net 4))
 (segment (start 132.05 59.85) (end 132.05 58.6) (width 0.4) (layer "F.Cu") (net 4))
 (segment (start 132.1 59.9) (end 132.05 59.85) (width 0.4) (layer "F.Cu") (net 4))
 (segment (start 132.6 59.9) (end 132.1 59.9) (width 0.4) (layer "F.Cu") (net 4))
 (segment (start 130.65 58.45) (end 130.4 58.2) (width 0.2) (layer "F.Cu") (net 4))
 (segment (start 130.45 59.45) (end 130.65 59.65) (width 0.2) (layer "F.Cu") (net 4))
 (segment (start 132.75 59.75) (end 132.6 59.9) (width 0.2) (layer "F.Cu") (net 4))
 (segment (start 132.6 59.9) (end 130.9 59.9) (width 0.2) (layer "F.Cu") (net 4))
 (segment (start 134.3 59.75) (end 132.75 59.75) (width 0.2) (layer "F.Cu") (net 4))
 (segment (start 132.6 59.9) (end 132.9 59.9) (width 0.2) (layer "F.Cu") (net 4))
 (segment (start 132.9 59.9) (end 133.15 59.65) (width 0.2) (layer "F.Cu") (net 4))
 (segment (start 130.4 58.2) (end 129.75 58.2) (width 0.2) (layer "F.Cu") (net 4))
 (segment (start 128.7 62.65) (end 128.7 60.75) (width 0.2) (layer "F.Cu") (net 3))
 (segment (start 128.7 60.75) (end 129.05 60.4) (width 0.2) (layer "F.Cu") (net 3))
 (segment (start 129.8 62.65) (end 128.7 62.65) (width 0.2) (layer "F.Cu") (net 3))
 (segment (start 139.8 70.4) (end 138.8 70.4) (width 0.4) (layer "F.Cu") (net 13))
 (segment (start 138.8 70.4) (end 138.6 70.6) (width 0.4) (layer "F.Cu") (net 13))
 (segment (start 138.6 70.6) (end 138.6 72.8) (width 0.4) (layer "F.Cu") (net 13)))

